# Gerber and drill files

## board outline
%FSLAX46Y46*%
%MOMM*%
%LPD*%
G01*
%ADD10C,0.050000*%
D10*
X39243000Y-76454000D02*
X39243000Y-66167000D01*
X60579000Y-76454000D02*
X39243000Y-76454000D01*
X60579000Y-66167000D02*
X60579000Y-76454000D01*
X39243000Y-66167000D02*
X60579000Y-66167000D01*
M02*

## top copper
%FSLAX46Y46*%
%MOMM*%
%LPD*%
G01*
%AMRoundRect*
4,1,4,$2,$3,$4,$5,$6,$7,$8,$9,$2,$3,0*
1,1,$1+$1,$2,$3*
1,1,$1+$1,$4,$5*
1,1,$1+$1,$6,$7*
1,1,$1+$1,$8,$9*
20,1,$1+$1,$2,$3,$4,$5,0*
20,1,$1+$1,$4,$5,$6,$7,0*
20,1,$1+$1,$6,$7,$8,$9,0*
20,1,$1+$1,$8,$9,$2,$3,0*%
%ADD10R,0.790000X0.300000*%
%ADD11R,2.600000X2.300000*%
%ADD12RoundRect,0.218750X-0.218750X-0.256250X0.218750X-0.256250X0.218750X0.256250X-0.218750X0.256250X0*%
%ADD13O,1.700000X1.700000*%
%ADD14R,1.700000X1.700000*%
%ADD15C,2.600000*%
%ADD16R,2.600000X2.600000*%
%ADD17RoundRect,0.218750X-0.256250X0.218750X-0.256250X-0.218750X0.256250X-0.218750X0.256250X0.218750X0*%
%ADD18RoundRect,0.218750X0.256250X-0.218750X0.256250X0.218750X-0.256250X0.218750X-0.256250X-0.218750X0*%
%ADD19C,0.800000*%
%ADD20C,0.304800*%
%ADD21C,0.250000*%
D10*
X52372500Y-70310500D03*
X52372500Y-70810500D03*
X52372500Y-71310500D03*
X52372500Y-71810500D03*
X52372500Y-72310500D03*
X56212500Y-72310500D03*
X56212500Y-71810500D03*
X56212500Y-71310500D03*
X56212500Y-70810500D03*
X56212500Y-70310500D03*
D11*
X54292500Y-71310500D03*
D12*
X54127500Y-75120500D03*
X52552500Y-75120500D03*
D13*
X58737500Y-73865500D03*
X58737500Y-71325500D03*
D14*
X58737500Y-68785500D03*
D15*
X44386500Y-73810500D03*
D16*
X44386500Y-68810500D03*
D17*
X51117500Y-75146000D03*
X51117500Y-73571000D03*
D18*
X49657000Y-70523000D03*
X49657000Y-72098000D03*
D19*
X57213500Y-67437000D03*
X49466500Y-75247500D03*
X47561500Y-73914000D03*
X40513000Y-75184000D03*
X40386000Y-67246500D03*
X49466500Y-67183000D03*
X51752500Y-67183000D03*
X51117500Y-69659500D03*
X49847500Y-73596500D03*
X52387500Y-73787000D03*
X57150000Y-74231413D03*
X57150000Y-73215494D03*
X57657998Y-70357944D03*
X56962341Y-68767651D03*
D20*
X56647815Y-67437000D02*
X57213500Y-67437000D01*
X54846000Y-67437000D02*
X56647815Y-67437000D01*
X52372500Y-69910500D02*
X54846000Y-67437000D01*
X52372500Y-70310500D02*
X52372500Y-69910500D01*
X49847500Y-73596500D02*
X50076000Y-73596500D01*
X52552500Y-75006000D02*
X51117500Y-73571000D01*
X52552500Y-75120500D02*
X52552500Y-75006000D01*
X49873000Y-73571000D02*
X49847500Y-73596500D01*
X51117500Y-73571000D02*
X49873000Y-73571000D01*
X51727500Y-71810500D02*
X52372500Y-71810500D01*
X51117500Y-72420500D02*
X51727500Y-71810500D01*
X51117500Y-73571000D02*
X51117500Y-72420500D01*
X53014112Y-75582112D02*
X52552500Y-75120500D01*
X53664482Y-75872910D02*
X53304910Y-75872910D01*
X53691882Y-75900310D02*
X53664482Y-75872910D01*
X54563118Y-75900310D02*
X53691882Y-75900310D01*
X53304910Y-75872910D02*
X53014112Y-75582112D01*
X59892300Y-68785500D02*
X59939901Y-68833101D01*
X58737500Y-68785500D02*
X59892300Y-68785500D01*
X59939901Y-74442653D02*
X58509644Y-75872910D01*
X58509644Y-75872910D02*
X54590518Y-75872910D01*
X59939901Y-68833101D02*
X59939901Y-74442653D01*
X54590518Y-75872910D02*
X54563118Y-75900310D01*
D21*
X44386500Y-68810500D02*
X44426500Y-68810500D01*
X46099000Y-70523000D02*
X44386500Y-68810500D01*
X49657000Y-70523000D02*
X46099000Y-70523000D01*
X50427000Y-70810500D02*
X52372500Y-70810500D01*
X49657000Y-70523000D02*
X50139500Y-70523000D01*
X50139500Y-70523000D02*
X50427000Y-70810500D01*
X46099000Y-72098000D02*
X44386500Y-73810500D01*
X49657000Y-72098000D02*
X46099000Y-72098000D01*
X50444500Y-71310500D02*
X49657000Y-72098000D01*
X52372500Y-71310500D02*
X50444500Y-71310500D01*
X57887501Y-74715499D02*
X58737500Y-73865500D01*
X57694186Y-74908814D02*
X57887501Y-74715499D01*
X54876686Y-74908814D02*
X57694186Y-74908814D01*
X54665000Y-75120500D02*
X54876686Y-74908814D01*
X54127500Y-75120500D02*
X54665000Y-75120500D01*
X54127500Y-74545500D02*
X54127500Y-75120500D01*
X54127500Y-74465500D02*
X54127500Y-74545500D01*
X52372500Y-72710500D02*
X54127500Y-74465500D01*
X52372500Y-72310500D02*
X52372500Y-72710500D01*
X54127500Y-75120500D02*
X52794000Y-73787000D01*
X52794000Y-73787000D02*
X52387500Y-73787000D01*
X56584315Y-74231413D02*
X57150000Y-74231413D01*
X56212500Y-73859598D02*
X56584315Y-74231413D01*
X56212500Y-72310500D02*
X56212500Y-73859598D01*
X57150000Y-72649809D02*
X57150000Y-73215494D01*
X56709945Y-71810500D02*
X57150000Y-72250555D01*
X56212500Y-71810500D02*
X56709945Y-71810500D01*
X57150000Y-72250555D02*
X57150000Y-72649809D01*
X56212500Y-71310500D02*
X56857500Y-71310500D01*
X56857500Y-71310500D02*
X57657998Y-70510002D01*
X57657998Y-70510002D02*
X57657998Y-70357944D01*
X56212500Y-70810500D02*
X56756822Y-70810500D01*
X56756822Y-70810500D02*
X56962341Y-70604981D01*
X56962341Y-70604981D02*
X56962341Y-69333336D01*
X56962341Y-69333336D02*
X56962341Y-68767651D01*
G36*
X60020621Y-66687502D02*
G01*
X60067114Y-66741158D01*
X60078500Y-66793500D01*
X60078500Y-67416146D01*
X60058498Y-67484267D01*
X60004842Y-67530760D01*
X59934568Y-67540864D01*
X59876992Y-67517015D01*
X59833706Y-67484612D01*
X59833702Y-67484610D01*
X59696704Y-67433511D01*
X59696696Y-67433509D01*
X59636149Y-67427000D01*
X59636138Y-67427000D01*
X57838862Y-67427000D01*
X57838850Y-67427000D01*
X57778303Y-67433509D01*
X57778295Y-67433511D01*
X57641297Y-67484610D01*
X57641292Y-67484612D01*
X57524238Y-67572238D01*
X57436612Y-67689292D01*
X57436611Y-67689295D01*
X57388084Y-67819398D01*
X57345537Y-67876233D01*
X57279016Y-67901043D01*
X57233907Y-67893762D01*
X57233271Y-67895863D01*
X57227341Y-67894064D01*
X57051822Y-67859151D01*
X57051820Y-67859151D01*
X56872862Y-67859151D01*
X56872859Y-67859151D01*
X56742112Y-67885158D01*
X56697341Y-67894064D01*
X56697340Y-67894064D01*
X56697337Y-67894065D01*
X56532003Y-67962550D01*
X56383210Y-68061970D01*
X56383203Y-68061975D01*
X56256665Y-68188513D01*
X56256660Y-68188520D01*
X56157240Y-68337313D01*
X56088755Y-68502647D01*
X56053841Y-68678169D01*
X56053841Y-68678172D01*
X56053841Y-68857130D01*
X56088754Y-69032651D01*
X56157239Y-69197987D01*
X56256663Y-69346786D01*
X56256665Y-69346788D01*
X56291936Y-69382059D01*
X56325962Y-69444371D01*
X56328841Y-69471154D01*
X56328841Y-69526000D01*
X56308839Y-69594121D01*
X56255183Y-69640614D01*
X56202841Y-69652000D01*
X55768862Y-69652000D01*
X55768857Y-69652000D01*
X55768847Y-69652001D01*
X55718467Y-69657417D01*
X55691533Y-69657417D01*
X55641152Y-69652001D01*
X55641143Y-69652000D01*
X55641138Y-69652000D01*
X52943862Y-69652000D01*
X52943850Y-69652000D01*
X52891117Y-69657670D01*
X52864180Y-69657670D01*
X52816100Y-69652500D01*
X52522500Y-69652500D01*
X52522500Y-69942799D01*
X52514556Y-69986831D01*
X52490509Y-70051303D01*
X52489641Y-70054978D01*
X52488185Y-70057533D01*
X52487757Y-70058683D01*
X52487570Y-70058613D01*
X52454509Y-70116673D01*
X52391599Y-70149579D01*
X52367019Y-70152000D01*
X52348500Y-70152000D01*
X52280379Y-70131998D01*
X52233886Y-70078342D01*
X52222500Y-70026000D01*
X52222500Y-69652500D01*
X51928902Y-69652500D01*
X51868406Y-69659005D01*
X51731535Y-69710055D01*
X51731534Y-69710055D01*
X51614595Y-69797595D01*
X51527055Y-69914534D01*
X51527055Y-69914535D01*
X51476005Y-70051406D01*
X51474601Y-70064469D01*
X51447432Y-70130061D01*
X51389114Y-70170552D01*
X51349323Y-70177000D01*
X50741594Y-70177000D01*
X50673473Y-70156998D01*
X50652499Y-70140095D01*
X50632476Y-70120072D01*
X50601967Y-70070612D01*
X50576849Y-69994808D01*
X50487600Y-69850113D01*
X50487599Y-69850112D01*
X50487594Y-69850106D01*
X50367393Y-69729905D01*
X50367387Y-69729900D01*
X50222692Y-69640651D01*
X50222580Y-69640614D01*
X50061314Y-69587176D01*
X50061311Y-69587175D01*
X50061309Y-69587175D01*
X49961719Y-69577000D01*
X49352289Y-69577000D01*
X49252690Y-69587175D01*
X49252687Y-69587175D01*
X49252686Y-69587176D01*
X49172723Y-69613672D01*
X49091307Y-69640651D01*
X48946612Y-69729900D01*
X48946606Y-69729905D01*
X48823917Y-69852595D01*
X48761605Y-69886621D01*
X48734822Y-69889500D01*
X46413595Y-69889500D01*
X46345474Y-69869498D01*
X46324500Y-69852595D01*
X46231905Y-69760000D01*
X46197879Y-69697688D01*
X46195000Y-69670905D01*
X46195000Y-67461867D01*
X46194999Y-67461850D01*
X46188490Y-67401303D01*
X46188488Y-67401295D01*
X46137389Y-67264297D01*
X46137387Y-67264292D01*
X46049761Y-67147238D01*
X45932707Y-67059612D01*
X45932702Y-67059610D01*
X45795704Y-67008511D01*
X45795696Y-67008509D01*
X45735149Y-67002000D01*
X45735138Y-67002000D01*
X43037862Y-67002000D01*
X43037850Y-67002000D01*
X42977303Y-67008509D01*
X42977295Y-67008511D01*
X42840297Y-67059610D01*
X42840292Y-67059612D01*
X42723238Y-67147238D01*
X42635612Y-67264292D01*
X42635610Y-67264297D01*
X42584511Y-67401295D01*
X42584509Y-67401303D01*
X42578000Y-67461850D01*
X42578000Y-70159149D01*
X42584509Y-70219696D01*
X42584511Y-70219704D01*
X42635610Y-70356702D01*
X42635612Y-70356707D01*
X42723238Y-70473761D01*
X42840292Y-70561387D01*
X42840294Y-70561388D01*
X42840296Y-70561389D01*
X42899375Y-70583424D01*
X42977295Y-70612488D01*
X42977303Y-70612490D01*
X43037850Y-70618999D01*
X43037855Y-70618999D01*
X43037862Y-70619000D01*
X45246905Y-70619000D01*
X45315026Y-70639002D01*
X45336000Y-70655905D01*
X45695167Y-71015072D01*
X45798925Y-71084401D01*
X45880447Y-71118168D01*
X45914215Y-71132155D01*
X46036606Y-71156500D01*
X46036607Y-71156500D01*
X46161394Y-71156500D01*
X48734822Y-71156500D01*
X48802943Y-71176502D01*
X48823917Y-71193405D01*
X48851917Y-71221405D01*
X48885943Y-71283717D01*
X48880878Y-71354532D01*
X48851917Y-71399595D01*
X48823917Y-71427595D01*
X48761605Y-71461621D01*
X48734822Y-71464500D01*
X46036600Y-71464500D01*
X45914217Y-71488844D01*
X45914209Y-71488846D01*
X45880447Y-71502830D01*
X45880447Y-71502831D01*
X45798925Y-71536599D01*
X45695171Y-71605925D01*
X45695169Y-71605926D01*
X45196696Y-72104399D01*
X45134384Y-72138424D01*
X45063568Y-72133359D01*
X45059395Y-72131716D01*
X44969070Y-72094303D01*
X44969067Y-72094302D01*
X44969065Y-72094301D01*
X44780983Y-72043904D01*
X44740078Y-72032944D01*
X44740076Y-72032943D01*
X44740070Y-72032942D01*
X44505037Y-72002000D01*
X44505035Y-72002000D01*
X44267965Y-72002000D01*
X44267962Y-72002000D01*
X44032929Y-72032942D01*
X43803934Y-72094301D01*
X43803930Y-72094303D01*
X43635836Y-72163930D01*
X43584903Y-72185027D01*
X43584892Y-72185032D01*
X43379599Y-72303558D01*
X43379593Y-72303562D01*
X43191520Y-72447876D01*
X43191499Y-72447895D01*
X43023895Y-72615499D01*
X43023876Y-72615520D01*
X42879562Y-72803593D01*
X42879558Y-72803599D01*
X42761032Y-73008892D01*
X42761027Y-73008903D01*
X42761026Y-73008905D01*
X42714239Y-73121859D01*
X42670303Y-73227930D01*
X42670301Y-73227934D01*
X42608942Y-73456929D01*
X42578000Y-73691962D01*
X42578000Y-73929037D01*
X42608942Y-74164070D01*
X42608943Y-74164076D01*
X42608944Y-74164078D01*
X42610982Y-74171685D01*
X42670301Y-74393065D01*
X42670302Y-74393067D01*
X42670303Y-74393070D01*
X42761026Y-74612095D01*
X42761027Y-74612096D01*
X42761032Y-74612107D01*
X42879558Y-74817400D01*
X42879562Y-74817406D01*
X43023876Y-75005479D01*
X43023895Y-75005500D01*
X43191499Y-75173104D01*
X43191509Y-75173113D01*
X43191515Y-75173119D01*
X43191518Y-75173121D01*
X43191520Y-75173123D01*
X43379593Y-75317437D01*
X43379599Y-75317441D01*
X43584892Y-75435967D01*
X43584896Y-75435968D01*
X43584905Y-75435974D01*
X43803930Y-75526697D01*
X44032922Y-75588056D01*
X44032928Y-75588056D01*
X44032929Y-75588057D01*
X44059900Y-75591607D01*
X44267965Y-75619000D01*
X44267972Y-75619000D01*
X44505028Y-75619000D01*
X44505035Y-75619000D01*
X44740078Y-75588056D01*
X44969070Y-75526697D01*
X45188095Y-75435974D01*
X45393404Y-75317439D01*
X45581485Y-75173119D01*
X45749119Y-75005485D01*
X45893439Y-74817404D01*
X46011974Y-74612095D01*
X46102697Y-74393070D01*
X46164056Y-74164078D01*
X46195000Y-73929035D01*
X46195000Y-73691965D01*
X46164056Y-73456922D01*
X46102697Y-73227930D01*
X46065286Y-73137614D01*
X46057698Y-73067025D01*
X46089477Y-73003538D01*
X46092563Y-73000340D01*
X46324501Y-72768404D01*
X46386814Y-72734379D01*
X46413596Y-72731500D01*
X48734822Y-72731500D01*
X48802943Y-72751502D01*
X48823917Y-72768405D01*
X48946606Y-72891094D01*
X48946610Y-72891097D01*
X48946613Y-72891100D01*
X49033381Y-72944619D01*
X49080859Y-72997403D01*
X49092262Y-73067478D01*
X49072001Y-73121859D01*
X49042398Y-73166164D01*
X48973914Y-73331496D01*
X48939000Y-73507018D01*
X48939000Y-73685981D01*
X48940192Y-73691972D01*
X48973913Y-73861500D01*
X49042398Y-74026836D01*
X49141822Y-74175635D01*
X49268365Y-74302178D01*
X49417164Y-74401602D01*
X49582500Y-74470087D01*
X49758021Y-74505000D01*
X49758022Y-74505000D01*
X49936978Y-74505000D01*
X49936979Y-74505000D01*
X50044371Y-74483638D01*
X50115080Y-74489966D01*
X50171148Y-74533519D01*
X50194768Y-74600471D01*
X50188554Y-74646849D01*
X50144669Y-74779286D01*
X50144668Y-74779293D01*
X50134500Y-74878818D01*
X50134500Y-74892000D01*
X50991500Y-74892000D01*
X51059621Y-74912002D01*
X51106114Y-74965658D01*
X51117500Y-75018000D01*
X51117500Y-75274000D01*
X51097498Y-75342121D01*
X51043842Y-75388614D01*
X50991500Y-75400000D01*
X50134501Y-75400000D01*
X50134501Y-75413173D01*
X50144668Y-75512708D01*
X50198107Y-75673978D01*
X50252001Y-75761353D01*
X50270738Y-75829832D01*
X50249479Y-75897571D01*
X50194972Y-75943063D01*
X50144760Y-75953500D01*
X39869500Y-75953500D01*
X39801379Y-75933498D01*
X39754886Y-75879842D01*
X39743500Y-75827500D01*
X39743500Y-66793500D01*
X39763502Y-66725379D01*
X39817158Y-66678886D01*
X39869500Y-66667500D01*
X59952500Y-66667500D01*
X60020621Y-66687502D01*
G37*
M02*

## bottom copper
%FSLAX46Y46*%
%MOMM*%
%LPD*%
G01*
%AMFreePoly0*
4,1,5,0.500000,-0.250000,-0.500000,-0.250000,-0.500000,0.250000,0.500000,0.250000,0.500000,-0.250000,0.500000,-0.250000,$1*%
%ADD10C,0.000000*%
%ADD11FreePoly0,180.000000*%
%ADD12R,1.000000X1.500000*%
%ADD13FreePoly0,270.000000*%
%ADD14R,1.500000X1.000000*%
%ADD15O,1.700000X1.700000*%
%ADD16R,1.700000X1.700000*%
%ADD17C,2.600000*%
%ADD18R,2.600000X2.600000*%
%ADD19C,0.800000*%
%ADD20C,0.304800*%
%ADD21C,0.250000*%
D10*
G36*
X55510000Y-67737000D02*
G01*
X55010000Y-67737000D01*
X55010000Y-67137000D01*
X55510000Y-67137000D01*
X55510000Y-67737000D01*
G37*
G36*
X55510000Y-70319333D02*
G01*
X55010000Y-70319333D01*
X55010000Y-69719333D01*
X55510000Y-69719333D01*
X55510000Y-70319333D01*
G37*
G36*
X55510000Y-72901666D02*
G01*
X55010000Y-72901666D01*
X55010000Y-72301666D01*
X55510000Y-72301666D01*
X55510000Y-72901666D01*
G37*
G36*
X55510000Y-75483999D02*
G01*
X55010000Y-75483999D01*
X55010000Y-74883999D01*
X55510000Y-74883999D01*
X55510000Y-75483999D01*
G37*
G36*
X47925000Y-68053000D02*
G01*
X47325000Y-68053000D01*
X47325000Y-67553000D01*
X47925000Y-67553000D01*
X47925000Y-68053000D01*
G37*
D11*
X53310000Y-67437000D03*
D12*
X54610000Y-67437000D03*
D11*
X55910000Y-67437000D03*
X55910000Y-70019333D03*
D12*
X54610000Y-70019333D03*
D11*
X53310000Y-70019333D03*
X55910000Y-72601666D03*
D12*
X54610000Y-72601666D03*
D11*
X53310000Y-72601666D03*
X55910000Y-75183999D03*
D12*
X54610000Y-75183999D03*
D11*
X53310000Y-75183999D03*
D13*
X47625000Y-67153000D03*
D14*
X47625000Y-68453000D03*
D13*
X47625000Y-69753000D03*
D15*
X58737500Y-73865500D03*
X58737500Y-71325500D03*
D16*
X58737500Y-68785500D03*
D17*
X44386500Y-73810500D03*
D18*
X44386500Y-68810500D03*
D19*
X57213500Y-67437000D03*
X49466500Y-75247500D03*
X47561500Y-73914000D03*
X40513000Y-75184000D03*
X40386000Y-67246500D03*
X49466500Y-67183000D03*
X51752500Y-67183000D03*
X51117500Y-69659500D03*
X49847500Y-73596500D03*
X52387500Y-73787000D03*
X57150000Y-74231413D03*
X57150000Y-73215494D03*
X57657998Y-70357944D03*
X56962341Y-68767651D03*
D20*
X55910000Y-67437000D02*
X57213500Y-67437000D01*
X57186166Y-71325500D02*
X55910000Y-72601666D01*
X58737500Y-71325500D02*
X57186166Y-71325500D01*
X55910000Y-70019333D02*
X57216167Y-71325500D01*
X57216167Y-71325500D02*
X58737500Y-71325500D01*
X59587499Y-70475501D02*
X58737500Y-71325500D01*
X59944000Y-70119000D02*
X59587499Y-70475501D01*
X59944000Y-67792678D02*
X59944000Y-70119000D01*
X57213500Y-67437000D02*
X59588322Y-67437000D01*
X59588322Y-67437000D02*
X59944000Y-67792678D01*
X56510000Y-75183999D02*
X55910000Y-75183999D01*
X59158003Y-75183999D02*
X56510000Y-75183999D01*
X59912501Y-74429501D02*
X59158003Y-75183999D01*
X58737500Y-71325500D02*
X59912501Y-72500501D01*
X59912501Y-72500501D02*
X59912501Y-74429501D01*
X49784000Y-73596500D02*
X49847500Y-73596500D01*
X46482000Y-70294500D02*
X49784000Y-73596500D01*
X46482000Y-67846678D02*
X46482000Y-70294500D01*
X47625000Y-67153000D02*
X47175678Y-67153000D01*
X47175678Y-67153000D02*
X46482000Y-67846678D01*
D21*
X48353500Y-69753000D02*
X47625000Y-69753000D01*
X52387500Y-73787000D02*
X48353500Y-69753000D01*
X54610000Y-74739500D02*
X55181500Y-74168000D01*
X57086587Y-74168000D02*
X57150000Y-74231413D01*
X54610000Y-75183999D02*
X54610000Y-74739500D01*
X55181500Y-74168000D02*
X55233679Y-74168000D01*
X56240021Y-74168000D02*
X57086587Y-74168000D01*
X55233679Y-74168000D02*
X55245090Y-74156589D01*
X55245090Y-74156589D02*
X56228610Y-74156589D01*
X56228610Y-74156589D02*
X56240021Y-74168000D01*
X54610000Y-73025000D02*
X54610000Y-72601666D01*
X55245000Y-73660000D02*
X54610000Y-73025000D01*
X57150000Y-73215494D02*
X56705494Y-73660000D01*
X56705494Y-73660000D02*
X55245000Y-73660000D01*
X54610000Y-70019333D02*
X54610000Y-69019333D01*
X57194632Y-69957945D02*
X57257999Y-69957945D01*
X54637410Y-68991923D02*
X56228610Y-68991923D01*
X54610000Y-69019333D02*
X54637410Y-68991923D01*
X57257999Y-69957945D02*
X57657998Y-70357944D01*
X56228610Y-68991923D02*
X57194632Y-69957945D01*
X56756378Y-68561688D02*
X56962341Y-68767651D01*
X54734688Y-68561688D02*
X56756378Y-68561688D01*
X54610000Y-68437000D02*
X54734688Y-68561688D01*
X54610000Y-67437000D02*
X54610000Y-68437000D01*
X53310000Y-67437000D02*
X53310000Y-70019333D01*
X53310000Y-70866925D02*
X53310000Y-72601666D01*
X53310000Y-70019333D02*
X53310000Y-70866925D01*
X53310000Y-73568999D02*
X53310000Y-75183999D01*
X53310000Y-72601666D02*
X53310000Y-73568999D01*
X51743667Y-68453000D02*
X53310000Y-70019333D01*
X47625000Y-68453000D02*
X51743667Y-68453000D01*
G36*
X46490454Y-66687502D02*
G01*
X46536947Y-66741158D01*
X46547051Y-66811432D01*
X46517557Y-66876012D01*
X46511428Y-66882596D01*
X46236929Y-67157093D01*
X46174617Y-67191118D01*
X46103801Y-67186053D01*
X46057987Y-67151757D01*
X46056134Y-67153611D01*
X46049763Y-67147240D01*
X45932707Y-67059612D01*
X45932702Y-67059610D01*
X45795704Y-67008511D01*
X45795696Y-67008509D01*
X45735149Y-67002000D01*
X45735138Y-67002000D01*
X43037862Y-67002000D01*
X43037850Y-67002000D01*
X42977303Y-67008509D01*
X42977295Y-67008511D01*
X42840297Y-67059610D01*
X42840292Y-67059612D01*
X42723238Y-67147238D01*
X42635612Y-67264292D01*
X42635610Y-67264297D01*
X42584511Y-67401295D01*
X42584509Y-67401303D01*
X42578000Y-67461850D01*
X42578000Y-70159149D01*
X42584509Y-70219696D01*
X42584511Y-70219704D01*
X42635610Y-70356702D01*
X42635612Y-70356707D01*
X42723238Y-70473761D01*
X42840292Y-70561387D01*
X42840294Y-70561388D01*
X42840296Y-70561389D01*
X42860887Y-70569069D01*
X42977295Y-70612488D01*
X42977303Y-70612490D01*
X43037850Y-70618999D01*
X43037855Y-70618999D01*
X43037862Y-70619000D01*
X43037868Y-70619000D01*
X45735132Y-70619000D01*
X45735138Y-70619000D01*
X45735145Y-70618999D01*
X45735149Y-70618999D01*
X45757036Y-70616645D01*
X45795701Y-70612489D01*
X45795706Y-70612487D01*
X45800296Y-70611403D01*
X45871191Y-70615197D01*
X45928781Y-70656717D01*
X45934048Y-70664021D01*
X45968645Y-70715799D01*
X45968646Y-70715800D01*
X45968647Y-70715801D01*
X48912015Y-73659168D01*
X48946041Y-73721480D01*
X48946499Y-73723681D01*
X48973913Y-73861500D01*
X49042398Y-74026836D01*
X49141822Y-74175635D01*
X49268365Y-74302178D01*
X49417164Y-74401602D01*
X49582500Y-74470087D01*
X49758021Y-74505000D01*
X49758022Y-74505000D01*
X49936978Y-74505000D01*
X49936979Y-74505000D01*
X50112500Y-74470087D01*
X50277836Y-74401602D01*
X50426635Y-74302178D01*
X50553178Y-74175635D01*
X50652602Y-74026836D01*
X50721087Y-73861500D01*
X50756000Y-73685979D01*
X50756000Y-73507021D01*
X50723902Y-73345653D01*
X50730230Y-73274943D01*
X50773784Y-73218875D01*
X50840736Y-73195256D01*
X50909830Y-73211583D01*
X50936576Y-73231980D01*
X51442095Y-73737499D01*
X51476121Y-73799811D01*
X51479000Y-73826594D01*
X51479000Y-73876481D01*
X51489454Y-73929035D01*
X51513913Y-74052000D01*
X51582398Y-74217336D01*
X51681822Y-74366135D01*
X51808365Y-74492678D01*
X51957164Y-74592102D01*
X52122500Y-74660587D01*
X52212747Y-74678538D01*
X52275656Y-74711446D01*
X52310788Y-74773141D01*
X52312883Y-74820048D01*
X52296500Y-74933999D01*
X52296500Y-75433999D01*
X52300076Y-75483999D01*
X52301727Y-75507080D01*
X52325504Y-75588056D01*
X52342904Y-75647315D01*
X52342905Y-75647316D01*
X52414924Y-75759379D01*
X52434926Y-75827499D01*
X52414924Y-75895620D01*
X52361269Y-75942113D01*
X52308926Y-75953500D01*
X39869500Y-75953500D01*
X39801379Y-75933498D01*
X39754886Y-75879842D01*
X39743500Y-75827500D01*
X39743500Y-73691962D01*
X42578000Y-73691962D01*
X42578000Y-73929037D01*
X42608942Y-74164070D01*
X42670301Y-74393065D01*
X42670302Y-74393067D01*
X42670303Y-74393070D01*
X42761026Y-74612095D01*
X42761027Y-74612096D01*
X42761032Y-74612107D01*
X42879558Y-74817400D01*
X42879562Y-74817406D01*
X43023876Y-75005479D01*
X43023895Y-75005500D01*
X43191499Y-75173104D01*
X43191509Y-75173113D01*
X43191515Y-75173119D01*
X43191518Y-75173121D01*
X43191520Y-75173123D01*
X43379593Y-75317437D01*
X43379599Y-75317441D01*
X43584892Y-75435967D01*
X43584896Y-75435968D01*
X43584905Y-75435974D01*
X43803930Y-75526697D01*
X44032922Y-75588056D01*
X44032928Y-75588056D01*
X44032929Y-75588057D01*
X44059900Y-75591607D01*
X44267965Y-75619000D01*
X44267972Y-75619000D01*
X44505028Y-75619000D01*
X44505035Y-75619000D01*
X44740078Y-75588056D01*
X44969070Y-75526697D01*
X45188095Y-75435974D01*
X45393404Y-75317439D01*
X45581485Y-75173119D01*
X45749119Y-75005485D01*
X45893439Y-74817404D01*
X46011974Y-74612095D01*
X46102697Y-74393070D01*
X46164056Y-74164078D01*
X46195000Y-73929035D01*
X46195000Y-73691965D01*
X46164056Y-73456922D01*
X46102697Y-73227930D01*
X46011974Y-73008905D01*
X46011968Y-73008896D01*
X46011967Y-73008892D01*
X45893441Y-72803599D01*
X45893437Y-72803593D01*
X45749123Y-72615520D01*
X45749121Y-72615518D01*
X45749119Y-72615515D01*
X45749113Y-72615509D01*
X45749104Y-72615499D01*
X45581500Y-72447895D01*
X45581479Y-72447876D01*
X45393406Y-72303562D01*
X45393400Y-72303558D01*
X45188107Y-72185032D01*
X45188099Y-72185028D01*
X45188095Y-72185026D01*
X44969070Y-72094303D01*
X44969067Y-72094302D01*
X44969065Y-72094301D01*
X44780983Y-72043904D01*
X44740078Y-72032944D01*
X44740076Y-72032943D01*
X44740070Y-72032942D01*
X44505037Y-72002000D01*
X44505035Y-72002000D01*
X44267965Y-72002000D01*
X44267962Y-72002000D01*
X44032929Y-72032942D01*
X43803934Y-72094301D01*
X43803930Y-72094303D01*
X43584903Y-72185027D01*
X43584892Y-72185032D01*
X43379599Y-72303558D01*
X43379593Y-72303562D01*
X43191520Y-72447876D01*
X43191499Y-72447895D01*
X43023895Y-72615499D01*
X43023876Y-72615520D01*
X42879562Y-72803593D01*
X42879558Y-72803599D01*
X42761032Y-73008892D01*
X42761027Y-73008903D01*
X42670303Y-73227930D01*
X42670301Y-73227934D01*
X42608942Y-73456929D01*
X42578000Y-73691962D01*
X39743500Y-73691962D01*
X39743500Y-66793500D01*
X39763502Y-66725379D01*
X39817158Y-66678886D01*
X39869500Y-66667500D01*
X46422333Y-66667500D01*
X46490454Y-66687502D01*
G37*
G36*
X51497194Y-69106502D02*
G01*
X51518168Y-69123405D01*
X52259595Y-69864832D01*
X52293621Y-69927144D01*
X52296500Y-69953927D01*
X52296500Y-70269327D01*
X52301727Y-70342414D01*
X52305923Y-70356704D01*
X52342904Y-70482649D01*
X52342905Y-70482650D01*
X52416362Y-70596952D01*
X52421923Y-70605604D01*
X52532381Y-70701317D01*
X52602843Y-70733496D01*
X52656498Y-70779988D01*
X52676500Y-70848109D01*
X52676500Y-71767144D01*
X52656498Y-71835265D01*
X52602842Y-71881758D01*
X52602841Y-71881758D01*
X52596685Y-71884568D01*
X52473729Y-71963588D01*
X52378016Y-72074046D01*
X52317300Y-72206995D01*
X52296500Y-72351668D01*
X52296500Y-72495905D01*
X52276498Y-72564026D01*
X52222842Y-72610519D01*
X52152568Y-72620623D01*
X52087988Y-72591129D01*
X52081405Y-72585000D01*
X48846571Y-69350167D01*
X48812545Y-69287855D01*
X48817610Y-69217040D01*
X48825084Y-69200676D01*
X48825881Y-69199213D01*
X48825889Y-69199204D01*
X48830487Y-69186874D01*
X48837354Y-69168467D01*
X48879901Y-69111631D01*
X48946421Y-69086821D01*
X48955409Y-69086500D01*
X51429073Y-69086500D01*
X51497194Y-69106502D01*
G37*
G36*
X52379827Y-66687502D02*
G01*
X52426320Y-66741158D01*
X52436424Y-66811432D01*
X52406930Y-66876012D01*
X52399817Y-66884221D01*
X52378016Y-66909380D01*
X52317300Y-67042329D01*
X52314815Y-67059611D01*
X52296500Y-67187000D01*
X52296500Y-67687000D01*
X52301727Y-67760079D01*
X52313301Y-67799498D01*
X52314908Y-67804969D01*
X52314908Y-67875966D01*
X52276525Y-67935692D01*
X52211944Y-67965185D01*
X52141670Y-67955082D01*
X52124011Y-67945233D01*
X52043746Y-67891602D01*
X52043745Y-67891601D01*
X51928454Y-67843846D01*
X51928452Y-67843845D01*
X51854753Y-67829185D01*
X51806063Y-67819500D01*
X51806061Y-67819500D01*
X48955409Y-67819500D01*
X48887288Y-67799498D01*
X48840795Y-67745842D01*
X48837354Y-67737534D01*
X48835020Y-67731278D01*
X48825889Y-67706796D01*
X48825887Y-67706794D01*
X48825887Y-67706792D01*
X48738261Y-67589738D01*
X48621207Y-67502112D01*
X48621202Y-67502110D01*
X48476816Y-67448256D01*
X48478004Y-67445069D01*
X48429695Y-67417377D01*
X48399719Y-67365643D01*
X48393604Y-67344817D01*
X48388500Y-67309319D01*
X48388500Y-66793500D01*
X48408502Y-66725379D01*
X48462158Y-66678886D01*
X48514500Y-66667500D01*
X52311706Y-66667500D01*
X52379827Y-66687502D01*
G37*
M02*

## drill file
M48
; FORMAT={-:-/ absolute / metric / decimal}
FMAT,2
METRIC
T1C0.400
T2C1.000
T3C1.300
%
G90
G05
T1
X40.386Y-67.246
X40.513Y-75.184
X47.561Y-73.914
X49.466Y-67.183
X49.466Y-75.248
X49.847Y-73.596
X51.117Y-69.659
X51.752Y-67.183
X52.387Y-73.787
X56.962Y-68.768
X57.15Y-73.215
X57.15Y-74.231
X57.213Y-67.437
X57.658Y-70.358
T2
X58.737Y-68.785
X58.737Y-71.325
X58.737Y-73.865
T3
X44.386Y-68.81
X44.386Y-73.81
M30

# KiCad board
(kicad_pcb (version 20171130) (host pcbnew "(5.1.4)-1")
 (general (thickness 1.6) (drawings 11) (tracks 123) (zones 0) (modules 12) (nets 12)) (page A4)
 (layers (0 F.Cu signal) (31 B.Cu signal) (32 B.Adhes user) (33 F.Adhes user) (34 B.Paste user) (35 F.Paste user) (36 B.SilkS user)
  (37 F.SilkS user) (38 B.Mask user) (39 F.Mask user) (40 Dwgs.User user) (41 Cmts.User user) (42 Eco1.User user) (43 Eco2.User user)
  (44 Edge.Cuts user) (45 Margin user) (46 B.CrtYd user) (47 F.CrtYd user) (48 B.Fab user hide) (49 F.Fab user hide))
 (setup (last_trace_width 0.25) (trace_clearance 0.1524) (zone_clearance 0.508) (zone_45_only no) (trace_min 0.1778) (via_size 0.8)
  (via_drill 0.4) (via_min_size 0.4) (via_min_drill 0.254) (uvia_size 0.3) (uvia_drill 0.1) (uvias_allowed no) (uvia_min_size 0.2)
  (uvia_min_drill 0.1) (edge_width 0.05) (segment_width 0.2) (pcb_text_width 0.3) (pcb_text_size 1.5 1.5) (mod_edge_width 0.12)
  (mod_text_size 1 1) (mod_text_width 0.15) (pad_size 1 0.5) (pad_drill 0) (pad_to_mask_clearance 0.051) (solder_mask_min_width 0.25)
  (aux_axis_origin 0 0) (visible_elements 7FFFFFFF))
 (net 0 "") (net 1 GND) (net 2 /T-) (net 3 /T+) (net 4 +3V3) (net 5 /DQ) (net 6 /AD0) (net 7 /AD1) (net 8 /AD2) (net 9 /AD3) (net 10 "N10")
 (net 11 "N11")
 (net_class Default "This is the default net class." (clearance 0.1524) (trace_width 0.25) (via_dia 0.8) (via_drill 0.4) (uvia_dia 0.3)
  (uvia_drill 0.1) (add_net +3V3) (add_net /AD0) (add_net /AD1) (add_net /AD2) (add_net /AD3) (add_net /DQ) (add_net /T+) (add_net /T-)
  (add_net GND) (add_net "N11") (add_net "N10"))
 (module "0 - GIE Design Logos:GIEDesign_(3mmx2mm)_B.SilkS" (layer F.Cu) (at 41.402 71.5645)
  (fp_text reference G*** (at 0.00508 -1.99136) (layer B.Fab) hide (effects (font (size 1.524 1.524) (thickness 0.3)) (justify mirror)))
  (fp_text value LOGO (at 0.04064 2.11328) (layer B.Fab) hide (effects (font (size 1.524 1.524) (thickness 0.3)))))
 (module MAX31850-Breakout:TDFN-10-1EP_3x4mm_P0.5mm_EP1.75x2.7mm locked (layer F.Cu) (at 54.2925 71.3105)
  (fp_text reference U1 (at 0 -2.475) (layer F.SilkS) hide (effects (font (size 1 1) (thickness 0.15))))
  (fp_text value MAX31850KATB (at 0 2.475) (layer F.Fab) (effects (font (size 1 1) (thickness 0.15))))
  (pad 1 smd rect (at -1.92 -1) (size 0.79 0.3) (layers F.Cu F.Paste F.Mask) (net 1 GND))
  (pad 2 smd rect (at -1.92 -0.5) (size 0.79 0.3) (layers F.Cu F.Paste F.Mask) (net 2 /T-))
  (pad 3 smd rect (at -1.92 0) (size 0.79 0.3) (layers F.Cu F.Paste F.Mask) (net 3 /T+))
  (pad 4 smd rect (at -1.92 0.5) (size 0.79 0.3) (layers F.Cu F.Paste F.Mask) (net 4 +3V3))
  (pad 5 smd rect (at -1.92 1) (size 0.79 0.3) (layers F.Cu F.Paste F.Mask) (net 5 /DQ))
  (pad 6 smd rect (at 1.92 1) (size 0.79 0.3) (layers F.Cu F.Paste F.Mask) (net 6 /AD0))
  (pad 7 smd rect (at 1.92 0.5) (size 0.79 0.3) (layers F.Cu F.Paste F.Mask) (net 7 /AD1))
  (pad 8 smd rect (at 1.92 0) (size 0.79 0.3) (layers F.Cu F.Paste F.Mask) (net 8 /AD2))
  (pad 9 smd rect (at 1.92 -0.5) (size 0.79 0.3) (layers F.Cu F.Paste F.Mask) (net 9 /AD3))
  (pad 10 smd rect (at 1.92 -1) (size 0.79 0.3) (layers F.Cu F.Paste F.Mask) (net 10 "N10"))
  (pad 11 smd rect (at 0 0) (size 2.6 2.3) (layers F.Cu F.Mask))
  (pad "" smd rect (at -0.3875 -0.62) (size 0.6 1.05) (layers F.Paste))
  (pad "" smd rect (at -0.3875 0.62) (size 0.6 1.05) (layers F.Paste))
  (pad "" smd rect (at 0.3875 -0.62) (size 0.6 1.05) (layers F.Paste))
  (pad "" smd rect (at 0.3875 0.62) (size 0.6 1.05) (layers F.Paste)))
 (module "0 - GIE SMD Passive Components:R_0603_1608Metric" (layer F.Cu) (at 53.34 75.1205)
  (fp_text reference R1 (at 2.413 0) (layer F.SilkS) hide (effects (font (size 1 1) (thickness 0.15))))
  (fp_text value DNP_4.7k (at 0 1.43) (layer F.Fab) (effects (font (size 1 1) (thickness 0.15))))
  (pad 2 smd roundrect (at 0.7875 0) (size 0.875 0.95) (layers F.Cu F.Paste F.Mask) (roundrect_rratio 0.25) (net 5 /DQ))
  (pad 1 smd roundrect (at -0.7875 0) (size 0.875 0.95) (layers F.Cu F.Paste F.Mask) (roundrect_rratio 0.25) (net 4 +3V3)))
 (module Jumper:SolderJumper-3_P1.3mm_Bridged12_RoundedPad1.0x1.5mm (layer B.Cu) (at 54.61 67.437 180)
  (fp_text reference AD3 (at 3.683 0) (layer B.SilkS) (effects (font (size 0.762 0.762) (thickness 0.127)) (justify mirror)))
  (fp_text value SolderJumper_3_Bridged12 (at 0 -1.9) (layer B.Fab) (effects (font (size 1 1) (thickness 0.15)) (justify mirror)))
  (fp_poly (pts (xy -0.9 0.3) (xy -0.4 0.3) (xy -0.4 -0.3) (xy -0.9 -0.3)) (layer B.Cu) (width 0))
  (pad 3 smd custom (at 1.3 0 180) (size 1 0.5) (layers B.Cu B.Mask) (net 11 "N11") (zone_connect 2)
   (options (clearance outline) (anchor rect)) (primitives))
  (pad 2 smd rect (at 0 0 180) (size 1 1.5) (layers B.Cu B.Mask) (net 9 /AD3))
  (pad 1 smd custom (at -1.3 0 180) (size 1 0.5) (layers B.Cu B.Mask) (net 1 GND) (zone_connect 2)
   (options (clearance convexhull) (anchor rect)) (primitives)))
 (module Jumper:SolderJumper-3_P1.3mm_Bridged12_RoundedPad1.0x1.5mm (layer B.Cu) (at 54.61 70.019333 180)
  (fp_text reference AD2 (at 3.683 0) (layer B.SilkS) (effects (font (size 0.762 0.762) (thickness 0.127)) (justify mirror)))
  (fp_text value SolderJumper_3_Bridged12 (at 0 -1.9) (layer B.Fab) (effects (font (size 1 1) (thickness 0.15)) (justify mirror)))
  (fp_poly (pts (xy -0.9 0.3) (xy -0.4 0.3) (xy -0.4 -0.3) (xy -0.9 -0.3)) (layer B.Cu) (width 0))
  (pad 1 smd custom (at -1.3 0 180) (size 1 0.5) (layers B.Cu B.Mask) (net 1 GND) (zone_connect 2)
   (options (clearance outline) (anchor rect)) (primitives))
  (pad 2 smd rect (at 0 0 180) (size 1 1.5) (layers B.Cu B.Mask) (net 8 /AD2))
  (pad 3 smd custom (at 1.3 0 180) (size 1 0.5) (layers B.Cu B.Mask) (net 11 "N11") (zone_connect 2)
   (options (clearance outline) (anchor rect)) (primitives)))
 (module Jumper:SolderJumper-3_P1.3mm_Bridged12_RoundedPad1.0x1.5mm (layer B.Cu) (at 54.61 72.601666 180)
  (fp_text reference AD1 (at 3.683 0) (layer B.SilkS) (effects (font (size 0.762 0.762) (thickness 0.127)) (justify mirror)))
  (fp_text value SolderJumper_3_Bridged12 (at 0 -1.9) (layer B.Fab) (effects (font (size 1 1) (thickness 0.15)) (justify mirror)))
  (fp_poly (pts (xy -0.9 0.3) (xy -0.4 0.3) (xy -0.4 -0.3) (xy -0.9 -0.3)) (layer B.Cu) (width 0))
  (pad 1 smd custom (at -1.3 0 180) (size 1 0.5) (layers B.Cu B.Mask) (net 1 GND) (zone_connect 2)
   (options (clearance outline) (anchor rect)) (primitives))
  (pad 2 smd rect (at 0 0 180) (size 1 1.5) (layers B.Cu B.Mask) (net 7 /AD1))
  (pad 3 smd custom (at 1.3 0 180) (size 1 0.5) (layers B.Cu B.Mask) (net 11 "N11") (zone_connect 2)
   (options (clearance outline) (anchor rect)) (primitives)))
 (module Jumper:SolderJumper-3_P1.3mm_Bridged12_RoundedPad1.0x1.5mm (layer B.Cu) (at 54.61 75.183999 180)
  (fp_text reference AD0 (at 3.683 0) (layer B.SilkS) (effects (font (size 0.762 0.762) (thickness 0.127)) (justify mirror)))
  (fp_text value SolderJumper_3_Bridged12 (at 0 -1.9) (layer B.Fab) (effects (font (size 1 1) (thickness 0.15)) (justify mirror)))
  (fp_poly (pts (xy -0.9 0.3) (xy -0.4 0.3) (xy -0.4 -0.3) (xy -0.9 -0.3)) (layer B.Cu) (width 0))
  (pad 1 smd custom (at -1.3 0 180) (size 1 0.5) (layers B.Cu B.Mask) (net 1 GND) (zone_connect 2)
   (options (clearance outline) (anchor rect)) (primitives))
  (pad 2 smd rect (at 0 0 180) (size 1 1.5) (layers B.Cu B.Mask) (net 6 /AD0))
  (pad 3 smd custom (at 1.3 0 180) (size 1 0.5) (layers B.Cu B.Mask) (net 11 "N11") (zone_connect 2)
   (options (clearance outline) (anchor rect)) (primitives)))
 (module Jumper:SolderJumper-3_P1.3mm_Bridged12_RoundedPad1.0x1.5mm (layer B.Cu) (at 47.625 68.453 270)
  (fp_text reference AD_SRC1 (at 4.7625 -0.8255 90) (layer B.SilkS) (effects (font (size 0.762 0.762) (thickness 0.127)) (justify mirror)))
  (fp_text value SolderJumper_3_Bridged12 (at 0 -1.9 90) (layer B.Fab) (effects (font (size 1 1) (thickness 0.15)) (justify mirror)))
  (fp_poly (pts (xy -0.9 0.3) (xy -0.4 0.3) (xy -0.4 -0.3) (xy -0.9 -0.3)) (layer B.Cu) (width 0))
  (pad 1 smd custom (at -1.3 0 270) (size 1 0.5) (layers B.Cu B.Mask) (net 4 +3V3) (zone_connect 2)
   (options (clearance outline) (anchor rect)) (primitives))
  (pad 2 smd rect (at 0 0 270) (size 1 1.5) (layers B.Cu B.Mask) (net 11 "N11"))
  (pad 3 smd custom (at 1.3 0 270) (size 1 0.5) (layers B.Cu B.Mask) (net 5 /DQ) (zone_connect 2)
   (options (clearance outline) (anchor rect)) (primitives)))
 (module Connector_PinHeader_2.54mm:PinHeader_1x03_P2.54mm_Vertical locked (layer F.Cu) (at 58.7375 68.7855)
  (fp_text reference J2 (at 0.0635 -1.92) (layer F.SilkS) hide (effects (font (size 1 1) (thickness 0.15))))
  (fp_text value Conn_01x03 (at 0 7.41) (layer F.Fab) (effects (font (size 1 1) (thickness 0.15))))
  (pad 3 thru_hole oval (at 0 5.08) (size 1.7 1.7) (drill 1) (layers *.Cu *.Mask) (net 5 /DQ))
  (pad 2 thru_hole oval (at 0 2.54) (size 1.7 1.7) (drill 1) (layers *.Cu *.Mask) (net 1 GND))
  (pad 1 thru_hole rect (at 0 0) (size 1.7 1.7) (drill 1) (layers *.Cu *.Mask) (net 4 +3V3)))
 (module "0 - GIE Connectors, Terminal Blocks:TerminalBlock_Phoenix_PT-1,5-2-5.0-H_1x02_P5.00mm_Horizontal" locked (layer F.Cu)
  (at 44.3865 68.8105 270)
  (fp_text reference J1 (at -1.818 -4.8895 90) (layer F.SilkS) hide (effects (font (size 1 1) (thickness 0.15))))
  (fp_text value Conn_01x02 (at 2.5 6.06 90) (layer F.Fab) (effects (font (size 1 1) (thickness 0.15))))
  (pad 2 thru_hole circle (at 5 0 270) (size 2.6 2.6) (drill 1.3) (layers *.Cu *.Mask) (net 3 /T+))
  (pad 1 thru_hole rect (at 0 0 270) (size 2.6 2.6) (drill 1.3) (layers *.Cu *.Mask) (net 2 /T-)))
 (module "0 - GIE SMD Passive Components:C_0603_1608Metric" (layer F.Cu) (at 51.1175 74.3585 270)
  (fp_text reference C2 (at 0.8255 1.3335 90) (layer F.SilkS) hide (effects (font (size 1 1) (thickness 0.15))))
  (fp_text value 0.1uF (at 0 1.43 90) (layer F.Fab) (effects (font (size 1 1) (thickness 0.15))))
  (pad 2 smd roundrect (at 0.7875 0 270) (size 0.875 0.95) (layers F.Cu F.Paste F.Mask) (roundrect_rratio 0.25) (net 1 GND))
  (pad 1 smd roundrect (at -0.7875 0 270) (size 0.875 0.95) (layers F.Cu F.Paste F.Mask) (roundrect_rratio 0.25) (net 4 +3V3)))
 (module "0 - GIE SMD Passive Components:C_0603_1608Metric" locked (layer F.Cu) (at 49.657 71.3105 90)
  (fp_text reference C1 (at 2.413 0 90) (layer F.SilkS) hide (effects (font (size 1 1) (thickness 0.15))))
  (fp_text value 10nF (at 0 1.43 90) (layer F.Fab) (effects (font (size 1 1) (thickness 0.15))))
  (pad 2 smd roundrect (at 0.7875 0 90) (size 0.875 0.95) (layers F.Cu F.Paste F.Mask) (roundrect_rratio 0.25) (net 2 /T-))
  (pad 1 smd roundrect (at -0.7875 0 90) (size 0.875 0.95) (layers F.Cu F.Paste F.Mask) (roundrect_rratio 0.25) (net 3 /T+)))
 (gr_line (start 39.243 76.454) (end 39.243 66.167) (layer Edge.Cuts) (width 0.05))
 (gr_line (start 60.579 76.454) (end 39.243 76.454) (layer Edge.Cuts) (width 0.05))
 (gr_line (start 60.579 66.167) (end 60.579 76.454) (layer Edge.Cuts) (width 0.05))
 (gr_line (start 39.243 66.167) (end 60.579 66.167) (layer Edge.Cuts) (width 0.05))
 (segment (start 55.91 67.437) (end 57.2135 67.437) (width 0.3048) (layer B.Cu) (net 1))
 (segment (start 57.186166 71.3255) (end 55.91 72.601666) (width 0.3048) (layer B.Cu) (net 1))
 (segment (start 58.7375 71.3255) (end 57.186166 71.3255) (width 0.3048) (layer B.Cu) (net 1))
 (segment (start 55.91 70.019333) (end 57.216167 71.3255) (width 0.3048) (layer B.Cu) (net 1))
 (segment (start 57.216167 71.3255) (end 58.7375 71.3255) (width 0.3048) (layer B.Cu) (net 1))
 (via (at 57.2135 67.437) (size 0.8) (drill 0.4) (layers F.Cu B.Cu) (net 1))
 (segment (start 56.647815 67.437) (end 57.2135 67.437) (width 0.3048) (layer F.Cu) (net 1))
 (segment (start 54.846 67.437) (end 56.647815 67.437) (width 0.3048) (layer F.Cu) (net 1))
 (segment (start 52.3725 69.9105) (end 54.846 67.437) (width 0.3048) (layer F.Cu) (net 1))
 (segment (start 52.3725 70.3105) (end 52.3725 69.9105) (width 0.3048) (layer F.Cu) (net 1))
 (via (at 49.4665 75.2475) (size 0.8) (drill 0.4) (layers F.Cu B.Cu) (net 1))
 (via (at 47.5615 73.914) (size 0.8) (drill 0.4) (layers F.Cu B.Cu) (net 1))
 (via (at 40.513 75.184) (size 0.8) (drill 0.4) (layers F.Cu B.Cu) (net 1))
 (via (at 40.386 67.2465) (size 0.8) (drill 0.4) (layers F.Cu B.Cu) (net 1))
 (via (at 49.4665 67.183) (size 0.8) (drill 0.4) (layers F.Cu B.Cu) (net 1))
 (via (at 51.7525 67.183) (size 0.8) (drill 0.4) (layers F.Cu B.Cu) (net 1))
 (via (at 51.1175 69.6595) (size 0.8) (drill 0.4) (layers F.Cu B.Cu) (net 1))
 (segment (start 59.587499 70.475501) (end 58.7375 71.3255) (width 0.3048) (layer B.Cu) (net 1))
 (segment (start 59.944 70.119) (end 59.587499 70.475501) (width 0.3048) (layer B.Cu) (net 1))
 (segment (start 59.944 67.792678) (end 59.944 70.119) (width 0.3048) (layer B.Cu) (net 1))
 (segment (start 57.2135 67.437) (end 59.588322 67.437) (width 0.3048) (layer B.Cu) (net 1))
 (segment (start 59.588322 67.437) (end 59.944 67.792678) (width 0.3048) (layer B.Cu) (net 1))
 (segment (start 56.51 75.183999) (end 55.91 75.183999) (width 0.3048) (layer B.Cu) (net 1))
 (segment (start 59.158003 75.183999) (end 56.51 75.183999) (width 0.3048) (layer B.Cu) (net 1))
 (segment (start 59.912501 74.429501) (end 59.158003 75.183999) (width 0.3048) (layer B.Cu) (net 1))
 (segment (start 58.7375 71.3255) (end 59.912501 72.500501) (width 0.3048) (layer B.Cu) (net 1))
 (segment (start 59.912501 72.500501) (end 59.912501 74.429501) (width 0.3048) (layer B.Cu) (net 1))
 (via (at 49.8475 73.5965) (size 0.8) (drill 0.4) (layers F.Cu B.Cu) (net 4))
 (segment (start 49.8475 73.5965) (end 50.076 73.5965) (width 0.3048) (layer F.Cu) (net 4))
 (segment (start 52.5525 75.006) (end 51.1175 73.571) (width 0.3048) (layer F.Cu) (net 4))
 (segment (start 52.5525 75.1205) (end 52.5525 75.006) (width 0.3048) (layer F.Cu) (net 4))
 (segment (start 49.873 73.571) (end 49.8475 73.5965) (width 0.3048) (layer F.Cu) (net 4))
 (segment (start 51.1175 73.571) (end 49.873 73.571) (width 0.3048) (layer F.Cu) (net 4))
 (segment (start 51.7275 71.8105) (end 52.3725 71.8105) (width 0.3048) (layer F.Cu) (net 4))
 (segment (start 51.1175 72.4205) (end 51.7275 71.8105) (width 0.3048) (layer F.Cu) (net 4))
 (segment (start 51.1175 73.571) (end 51.1175 72.4205) (width 0.3048) (layer F.Cu) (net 4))
 (segment (start 49.784 73.5965) (end 49.8475 73.5965) (width 0.3048) (layer B.Cu) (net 4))
 (segment (start 46.482 70.2945) (end 49.784 73.5965) (width 0.3048) (layer B.Cu) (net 4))
 (segment (start 46.482 67.846678) (end 46.482 70.2945) (width 0.3048) (layer B.Cu) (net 4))
 (segment (start 47.625 67.153) (end 47.175678 67.153) (width 0.3048) (layer B.Cu) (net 4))
 (segment (start 47.175678 67.153) (end 46.482 67.846678) (width 0.3048) (layer B.Cu) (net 4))
 (segment (start 53.014112 75.582112) (end 52.5525 75.1205) (width 0.3048) (layer F.Cu) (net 4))
 (segment (start 53.664482 75.87291) (end 53.30491 75.87291) (width 0.3048) (layer F.Cu) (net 4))
 (segment (start 53.691882 75.90031) (end 53.664482 75.87291) (width 0.3048) (layer F.Cu) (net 4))
 (segment (start 54.563118 75.90031) (end 53.691882 75.90031) (width 0.3048) (layer F.Cu) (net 4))
 (segment (start 53.30491 75.87291) (end 53.014112 75.582112) (width 0.3048) (layer F.Cu) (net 4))
 (segment (start 59.8923 68.7855) (end 59.939901 68.833101) (width 0.3048) (layer F.Cu) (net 4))
 (segment (start 58.7375 68.7855) (end 59.8923 68.7855) (width 0.3048) (layer F.Cu) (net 4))
 (segment (start 59.939901 74.442653) (end 58.509644 75.87291) (width 0.3048) (layer F.Cu) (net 4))
 (segment (start 58.509644 75.87291) (end 54.590518 75.87291) (width 0.3048) (layer F.Cu) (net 4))
 (segment (start 59.939901 68.833101) (end 59.939901 74.442653) (width 0.3048) (layer F.Cu) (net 4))
 (segment (start 54.590518 75.87291) (end 54.563118 75.90031) (width 0.3048) (layer F.Cu) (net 4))
 (segment (start 44.3865 68.8105) (end 44.4265 68.8105) (width 0.25) (layer F.Cu) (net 2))
 (segment (start 46.099 70.523) (end 44.3865 68.8105) (width 0.25) (layer F.Cu) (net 2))
 (segment (start 49.657 70.523) (end 46.099 70.523) (width 0.25) (layer F.Cu) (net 2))
 (segment (start 50.427 70.8105) (end 52.3725 70.8105) (width 0.25) (layer F.Cu) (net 2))
 (segment (start 49.657 70.523) (end 50.1395 70.523) (width 0.25) (layer F.Cu) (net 2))
 (segment (start 50.1395 70.523) (end 50.427 70.8105) (width 0.25) (layer F.Cu) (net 2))
 (segment (start 46.099 72.098) (end 44.3865 73.8105) (width 0.25) (layer F.Cu) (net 3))
 (segment (start 49.657 72.098) (end 46.099 72.098) (width 0.25) (layer F.Cu) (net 3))
 (segment (start 50.4445 71.3105) (end 49.657 72.098) (width 0.25) (layer F.Cu) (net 3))
 (segment (start 52.3725 71.3105) (end 50.4445 71.3105) (width 0.25) (layer F.Cu) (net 3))
 (segment (start 57.887501 74.715499) (end 58.7375 73.8655) (width 0.25) (layer F.Cu) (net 5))
 (segment (start 57.694186 74.908814) (end 57.887501 74.715499) (width 0.25) (layer F.Cu) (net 5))
 (segment (start 54.876686 74.908814) (end 57.694186 74.908814) (width 0.25) (layer F.Cu) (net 5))
 (segment (start 54.665 75.1205) (end 54.876686 74.908814) (width 0.25) (layer F.Cu) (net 5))
 (segment (start 54.1275 75.1205) (end 54.665 75.1205) (width 0.25) (layer F.Cu) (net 5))
 (segment (start 54.1275 74.5455) (end 54.1275 75.1205) (width 0.25) (layer F.Cu) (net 5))
 (segment (start 54.1275 74.4655) (end 54.1275 74.5455) (width 0.25) (layer F.Cu) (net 5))
 (segment (start 52.3725 72.7105) (end 54.1275 74.4655) (width 0.25) (layer F.Cu) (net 5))
 (segment (start 52.3725 72.3105) (end 52.3725 72.7105) (width 0.25) (layer F.Cu) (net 5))
 (via (at 52.3875 73.787) (size 0.8) (drill 0.4) (layers F.Cu B.Cu) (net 5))
 (segment (start 54.1275 75.1205) (end 52.794 73.787) (width 0.25) (layer F.Cu) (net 5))
 (segment (start 52.794 73.787) (end 52.3875 73.787) (width 0.25) (layer F.Cu) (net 5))
 (segment (start 48.3535 69.753) (end 47.625 69.753) (width 0.25) (layer B.Cu) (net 5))
 (segment (start 52.3875 73.787) (end 48.3535 69.753) (width 0.25) (layer B.Cu) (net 5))
 (via (at 57.15 74.231413) (size 0.8) (drill 0.4) (layers F.Cu B.Cu) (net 6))
 (segment (start 56.584315 74.231413) (end 57.15 74.231413) (width 0.25) (layer F.Cu) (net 6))
 (segment (start 56.2125 73.859598) (end 56.584315 74.231413) (width 0.25) (layer F.Cu) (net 6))
 (segment (start 56.2125 72.3105) (end 56.2125 73.859598) (width 0.25) (layer F.Cu) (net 6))
 (segment (start 54.61 74.7395) (end 55.1815 74.168) (width 0.25) (layer B.Cu) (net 6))
 (segment (start 57.086587 74.168) (end 57.15 74.231413) (width 0.25) (layer B.Cu) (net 6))
 (segment (start 54.61 75.183999) (end 54.61 74.7395) (width 0.25) (layer B.Cu) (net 6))
 (segment (start 55.1815 74.168) (end 55.233679 74.168) (width 0.25) (layer B.Cu) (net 6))
 (segment (start 56.240021 74.168) (end 57.086587 74.168) (width 0.25) (layer B.Cu) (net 6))
 (segment (start 55.233679 74.168) (end 55.24509 74.156589) (width 0.25) (layer B.Cu) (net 6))
 (segment (start 55.24509 74.156589) (end 56.22861 74.156589) (width 0.25) (layer B.Cu) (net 6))
 (segment (start 56.22861 74.156589) (end 56.240021 74.168) (width 0.25) (layer B.Cu) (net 6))
 (via (at 57.15 73.215494) (size 0.8) (drill 0.4) (layers F.Cu B.Cu) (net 7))
 (segment (start 57.15 72.649809) (end 57.15 73.215494) (width 0.25) (layer F.Cu) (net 7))
 (segment (start 56.709945 71.8105) (end 57.15 72.250555) (width 0.25) (layer F.Cu) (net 7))
 (segment (start 56.2125 71.8105) (end 56.709945 71.8105) (width 0.25) (layer F.Cu) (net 7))
 (segment (start 57.15 72.250555) (end 57.15 72.649809) (width 0.25) (layer F.Cu) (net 7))
 (segment (start 54.61 73.025) (end 54.61 72.601666) (width 0.25) (layer B.Cu) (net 7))
 (segment (start 55.245 73.66) (end 54.61 73.025) (width 0.25) (layer B.Cu) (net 7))
 (segment (start 57.15 73.215494) (end 56.705494 73.66) (width 0.25) (layer B.Cu) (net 7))
 (segment (start 56.705494 73.66) (end 55.245 73.66) (width 0.25) (layer B.Cu) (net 7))
 (segment (start 56.2125 71.3105) (end 56.8575 71.3105) (width 0.25) (layer F.Cu) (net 8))
 (via (at 57.657998 70.357944) (size 0.8) (drill 0.4) (layers F.Cu B.Cu) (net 8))
 (segment (start 56.8575 71.3105) (end 57.657998 70.510002) (width 0.25) (layer F.Cu) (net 8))
 (segment (start 57.657998 70.510002) (end 57.657998 70.357944) (width 0.25) (layer F.Cu) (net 8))
 (segment (start 54.61 70.019333) (end 54.61 69.019333) (width 0.25) (layer B.Cu) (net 8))
 (segment (start 57.194632 69.957945) (end 57.257999 69.957945) (width 0.25) (layer B.Cu) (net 8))
 (segment (start 54.63741 68.991923) (end 56.22861 68.991923) (width 0.25) (layer B.Cu) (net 8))
 (segment (start 54.61 69.019333) (end 54.63741 68.991923) (width 0.25) (layer B.Cu) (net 8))
 (segment (start 57.257999 69.957945) (end 57.657998 70.357944) (width 0.25) (layer B.Cu) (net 8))
 (segment (start 56.22861 68.991923) (end 57.194632 69.957945) (width 0.25) (layer B.Cu) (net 8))
 (via (at 56.962341 68.767651) (size 0.8) (drill 0.4) (layers F.Cu B.Cu) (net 9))
 (segment (start 56.2125 70.8105) (end 56.756822 70.8105) (width 0.25) (layer F.Cu) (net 9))
 (segment (start 56.756378 68.561688) (end 56.962341 68.767651) (width 0.25) (layer B.Cu) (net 9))
 (segment (start 54.734688 68.561688) (end 56.756378 68.561688) (width 0.25) (layer B.Cu) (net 9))
 (segment (start 54.61 68.437) (end 54.734688 68.561688) (width 0.25) (layer B.Cu) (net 9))
 (segment (start 54.61 67.437) (end 54.61 68.437) (width 0.25) (layer B.Cu) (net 9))
 (segment (start 56.756822 70.8105) (end 56.962341 70.604981) (width 0.25) (layer F.Cu) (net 9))
 (segment (start 56.962341 70.604981) (end 56.962341 69.333336) (width 0.25) (layer F.Cu) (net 9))
 (segment (start 56.962341 69.333336) (end 56.962341 68.767651) (width 0.25) (layer F.Cu) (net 9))
 (segment (start 53.31 67.437) (end 53.31 70.019333) (width 0.25) (layer B.Cu) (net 11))
 (segment (start 53.31 70.866925) (end 53.31 72.601666) (width 0.25) (layer B.Cu) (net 11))
 (segment (start 53.31 70.019333) (end 53.31 70.866925) (width 0.25) (layer B.Cu) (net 11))
 (segment (start 53.31 73.568999) (end 53.31 75.183999) (width 0.25) (layer B.Cu) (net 11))
 (segment (start 53.31 72.601666) (end 53.31 73.568999) (width 0.25) (layer B.Cu) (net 11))
 (segment (start 51.743667 68.453) (end 53.31 70.019333) (width 0.25) (layer B.Cu) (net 11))
 (segment (start 47.625 68.453) (end 51.743667 68.453) (width 0.25) (layer B.Cu) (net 11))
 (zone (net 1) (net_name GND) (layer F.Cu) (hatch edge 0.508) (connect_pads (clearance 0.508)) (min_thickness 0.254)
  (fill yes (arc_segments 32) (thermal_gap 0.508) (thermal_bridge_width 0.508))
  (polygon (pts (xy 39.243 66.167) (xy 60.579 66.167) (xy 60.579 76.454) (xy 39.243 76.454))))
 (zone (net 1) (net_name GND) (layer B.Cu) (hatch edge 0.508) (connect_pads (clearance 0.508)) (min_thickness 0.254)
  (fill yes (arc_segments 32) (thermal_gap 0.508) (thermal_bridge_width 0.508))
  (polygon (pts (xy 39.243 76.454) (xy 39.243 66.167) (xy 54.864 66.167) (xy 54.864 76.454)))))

